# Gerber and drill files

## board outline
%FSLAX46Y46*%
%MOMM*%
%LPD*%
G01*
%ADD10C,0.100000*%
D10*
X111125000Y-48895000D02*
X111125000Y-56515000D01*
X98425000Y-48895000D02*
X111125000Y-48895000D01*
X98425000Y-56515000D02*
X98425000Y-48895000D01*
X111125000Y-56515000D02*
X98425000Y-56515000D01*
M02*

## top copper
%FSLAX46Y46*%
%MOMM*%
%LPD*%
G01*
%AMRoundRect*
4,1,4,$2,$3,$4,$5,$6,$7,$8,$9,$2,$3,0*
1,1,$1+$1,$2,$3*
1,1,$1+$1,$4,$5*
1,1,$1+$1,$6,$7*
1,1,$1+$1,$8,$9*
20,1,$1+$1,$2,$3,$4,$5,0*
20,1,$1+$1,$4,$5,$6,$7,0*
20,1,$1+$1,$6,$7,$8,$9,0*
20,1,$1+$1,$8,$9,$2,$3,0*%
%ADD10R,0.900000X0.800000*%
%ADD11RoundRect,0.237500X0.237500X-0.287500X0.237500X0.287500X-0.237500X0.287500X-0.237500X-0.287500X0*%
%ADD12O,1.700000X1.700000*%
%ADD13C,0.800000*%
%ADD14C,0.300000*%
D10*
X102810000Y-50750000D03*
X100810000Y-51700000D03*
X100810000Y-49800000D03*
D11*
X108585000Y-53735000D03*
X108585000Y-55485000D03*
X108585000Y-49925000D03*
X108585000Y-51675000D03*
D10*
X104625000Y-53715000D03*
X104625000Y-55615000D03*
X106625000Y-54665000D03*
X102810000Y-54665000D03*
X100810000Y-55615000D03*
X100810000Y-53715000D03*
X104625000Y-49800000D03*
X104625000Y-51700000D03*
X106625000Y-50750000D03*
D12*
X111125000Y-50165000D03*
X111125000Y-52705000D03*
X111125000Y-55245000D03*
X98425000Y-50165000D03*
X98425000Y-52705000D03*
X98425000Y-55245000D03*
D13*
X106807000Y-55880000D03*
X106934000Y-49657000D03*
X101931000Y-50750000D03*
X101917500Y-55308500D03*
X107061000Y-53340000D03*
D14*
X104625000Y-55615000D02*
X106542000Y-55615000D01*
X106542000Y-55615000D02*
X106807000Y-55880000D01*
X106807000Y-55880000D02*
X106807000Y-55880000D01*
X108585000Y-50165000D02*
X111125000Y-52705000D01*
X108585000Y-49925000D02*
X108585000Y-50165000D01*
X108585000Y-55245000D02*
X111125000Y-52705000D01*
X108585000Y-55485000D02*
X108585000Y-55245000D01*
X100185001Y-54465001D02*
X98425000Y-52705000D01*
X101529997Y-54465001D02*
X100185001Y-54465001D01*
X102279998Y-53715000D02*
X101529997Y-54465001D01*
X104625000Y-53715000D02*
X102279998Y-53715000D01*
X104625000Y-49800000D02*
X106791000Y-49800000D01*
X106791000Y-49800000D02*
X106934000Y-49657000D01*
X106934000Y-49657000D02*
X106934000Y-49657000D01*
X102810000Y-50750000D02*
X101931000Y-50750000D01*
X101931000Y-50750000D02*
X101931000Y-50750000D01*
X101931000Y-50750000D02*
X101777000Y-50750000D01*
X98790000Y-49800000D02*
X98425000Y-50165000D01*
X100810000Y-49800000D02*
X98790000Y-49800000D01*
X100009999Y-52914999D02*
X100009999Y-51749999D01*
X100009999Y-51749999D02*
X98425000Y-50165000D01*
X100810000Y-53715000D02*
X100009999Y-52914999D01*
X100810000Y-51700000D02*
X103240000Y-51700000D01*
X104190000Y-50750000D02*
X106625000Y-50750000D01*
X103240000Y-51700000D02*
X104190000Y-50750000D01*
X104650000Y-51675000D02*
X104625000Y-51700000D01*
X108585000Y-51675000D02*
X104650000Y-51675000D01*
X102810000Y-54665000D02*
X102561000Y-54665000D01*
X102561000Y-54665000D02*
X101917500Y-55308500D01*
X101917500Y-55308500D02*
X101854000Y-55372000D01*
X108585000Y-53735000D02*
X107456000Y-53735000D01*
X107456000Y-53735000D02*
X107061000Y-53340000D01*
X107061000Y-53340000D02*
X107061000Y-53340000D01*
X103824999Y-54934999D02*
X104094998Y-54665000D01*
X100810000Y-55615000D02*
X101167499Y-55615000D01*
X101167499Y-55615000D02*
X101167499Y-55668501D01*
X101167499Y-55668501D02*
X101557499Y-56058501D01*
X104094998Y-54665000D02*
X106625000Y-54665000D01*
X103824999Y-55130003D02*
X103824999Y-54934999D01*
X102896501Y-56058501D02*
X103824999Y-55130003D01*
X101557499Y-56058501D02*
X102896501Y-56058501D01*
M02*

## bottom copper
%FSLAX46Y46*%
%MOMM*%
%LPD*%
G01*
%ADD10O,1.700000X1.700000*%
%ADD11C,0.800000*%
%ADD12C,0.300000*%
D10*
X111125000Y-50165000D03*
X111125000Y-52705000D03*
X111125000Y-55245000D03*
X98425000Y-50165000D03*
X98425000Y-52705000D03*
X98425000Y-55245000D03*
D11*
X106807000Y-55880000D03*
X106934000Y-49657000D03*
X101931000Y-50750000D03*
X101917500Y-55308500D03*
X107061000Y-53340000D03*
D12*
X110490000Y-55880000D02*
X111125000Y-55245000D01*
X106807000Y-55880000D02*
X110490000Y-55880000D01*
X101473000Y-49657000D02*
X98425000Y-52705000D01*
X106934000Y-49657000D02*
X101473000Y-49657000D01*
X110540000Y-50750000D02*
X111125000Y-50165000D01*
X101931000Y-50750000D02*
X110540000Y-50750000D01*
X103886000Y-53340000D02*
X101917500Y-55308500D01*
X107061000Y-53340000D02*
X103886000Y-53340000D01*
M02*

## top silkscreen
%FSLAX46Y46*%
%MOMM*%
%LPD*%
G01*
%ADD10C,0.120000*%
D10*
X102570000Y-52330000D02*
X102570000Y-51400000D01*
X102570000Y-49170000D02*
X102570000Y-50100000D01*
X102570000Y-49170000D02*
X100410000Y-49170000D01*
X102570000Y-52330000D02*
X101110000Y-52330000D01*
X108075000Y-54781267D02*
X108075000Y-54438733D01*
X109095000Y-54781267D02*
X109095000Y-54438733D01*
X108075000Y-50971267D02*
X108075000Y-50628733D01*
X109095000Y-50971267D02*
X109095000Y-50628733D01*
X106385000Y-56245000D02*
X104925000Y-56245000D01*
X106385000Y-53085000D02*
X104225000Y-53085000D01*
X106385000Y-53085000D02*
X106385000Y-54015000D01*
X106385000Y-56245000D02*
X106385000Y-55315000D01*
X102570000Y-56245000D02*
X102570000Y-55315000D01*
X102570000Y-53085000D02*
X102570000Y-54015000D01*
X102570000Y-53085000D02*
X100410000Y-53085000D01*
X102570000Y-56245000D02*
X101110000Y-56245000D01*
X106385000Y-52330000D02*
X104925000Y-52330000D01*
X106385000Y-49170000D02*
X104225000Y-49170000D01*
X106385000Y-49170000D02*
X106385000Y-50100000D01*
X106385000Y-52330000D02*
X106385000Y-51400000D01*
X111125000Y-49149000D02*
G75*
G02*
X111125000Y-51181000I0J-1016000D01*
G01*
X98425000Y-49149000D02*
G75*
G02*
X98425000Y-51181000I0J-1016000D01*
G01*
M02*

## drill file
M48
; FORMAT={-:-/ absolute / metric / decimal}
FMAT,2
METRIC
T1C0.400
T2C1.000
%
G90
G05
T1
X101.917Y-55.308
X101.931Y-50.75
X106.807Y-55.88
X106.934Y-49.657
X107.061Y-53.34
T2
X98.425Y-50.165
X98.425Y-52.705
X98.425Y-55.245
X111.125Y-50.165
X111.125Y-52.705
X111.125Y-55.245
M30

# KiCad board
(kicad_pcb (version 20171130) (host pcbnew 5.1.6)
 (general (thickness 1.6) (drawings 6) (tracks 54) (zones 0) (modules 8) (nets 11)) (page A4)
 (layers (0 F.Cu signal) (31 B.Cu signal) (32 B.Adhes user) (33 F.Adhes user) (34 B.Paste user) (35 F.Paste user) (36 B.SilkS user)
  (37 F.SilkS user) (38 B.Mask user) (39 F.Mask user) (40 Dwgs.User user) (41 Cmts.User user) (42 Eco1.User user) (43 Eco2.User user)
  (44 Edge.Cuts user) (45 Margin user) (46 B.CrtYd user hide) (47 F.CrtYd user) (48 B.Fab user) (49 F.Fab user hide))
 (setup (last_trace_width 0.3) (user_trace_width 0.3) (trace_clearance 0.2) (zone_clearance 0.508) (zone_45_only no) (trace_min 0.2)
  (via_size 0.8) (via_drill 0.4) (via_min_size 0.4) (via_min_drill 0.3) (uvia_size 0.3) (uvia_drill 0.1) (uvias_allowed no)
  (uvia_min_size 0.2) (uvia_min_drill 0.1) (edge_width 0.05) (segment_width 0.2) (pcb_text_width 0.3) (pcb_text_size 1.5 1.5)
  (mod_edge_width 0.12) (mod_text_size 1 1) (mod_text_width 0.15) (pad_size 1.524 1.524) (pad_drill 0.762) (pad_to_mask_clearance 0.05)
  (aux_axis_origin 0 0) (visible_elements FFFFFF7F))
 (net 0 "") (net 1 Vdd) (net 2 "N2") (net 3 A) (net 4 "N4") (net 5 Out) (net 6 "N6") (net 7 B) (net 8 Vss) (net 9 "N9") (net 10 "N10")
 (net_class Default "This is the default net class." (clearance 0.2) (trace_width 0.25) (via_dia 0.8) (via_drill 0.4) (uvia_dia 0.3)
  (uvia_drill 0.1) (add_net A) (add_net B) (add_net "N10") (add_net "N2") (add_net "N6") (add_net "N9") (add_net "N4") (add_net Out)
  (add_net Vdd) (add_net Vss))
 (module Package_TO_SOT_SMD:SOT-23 (layer F.Cu) (at 101.81 50.75)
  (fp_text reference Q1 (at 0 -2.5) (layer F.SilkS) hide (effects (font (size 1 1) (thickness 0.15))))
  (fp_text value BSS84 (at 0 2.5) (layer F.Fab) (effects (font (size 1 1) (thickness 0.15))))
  (fp_line (start 0.76 1.58) (end 0.76 0.65) (layer F.SilkS) (width 0.12))
  (fp_line (start 0.76 -1.58) (end 0.76 -0.65) (layer F.SilkS) (width 0.12))
  (fp_line (start 0.76 -1.58) (end -1.4 -1.58) (layer F.SilkS) (width 0.12))
  (fp_line (start 0.76 1.58) (end -0.7 1.58) (layer F.SilkS) (width 0.12))
  (pad 3 smd rect (at 1 0) (size 0.9 0.8) (layers F.Cu F.Paste F.Mask) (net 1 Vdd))
  (pad 2 smd rect (at -1 0.95) (size 0.9 0.8) (layers F.Cu F.Paste F.Mask) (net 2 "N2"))
  (pad 1 smd rect (at -1 -0.95) (size 0.9 0.8) (layers F.Cu F.Paste F.Mask) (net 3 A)))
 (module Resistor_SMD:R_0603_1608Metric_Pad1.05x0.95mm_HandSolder (layer F.Cu) (at 108.585 54.61 90)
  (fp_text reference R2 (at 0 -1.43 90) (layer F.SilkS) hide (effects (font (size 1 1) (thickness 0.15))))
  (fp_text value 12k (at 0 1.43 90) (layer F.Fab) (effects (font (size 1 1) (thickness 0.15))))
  (fp_line (start -0.171267 -0.51) (end 0.171267 -0.51) (layer F.SilkS) (width 0.12))
  (fp_line (start -0.171267 0.51) (end 0.171267 0.51) (layer F.SilkS) (width 0.12))
  (pad 2 smd roundrect (at 0.875 0 90) (size 1.05 0.95) (layers F.Cu F.Paste F.Mask) (roundrect_rratio 0.25) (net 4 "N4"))
  (pad 1 smd roundrect (at -0.875 0 90) (size 1.05 0.95) (layers F.Cu F.Paste F.Mask) (roundrect_rratio 0.25) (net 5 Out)))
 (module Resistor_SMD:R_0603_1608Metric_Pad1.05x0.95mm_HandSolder (layer F.Cu) (at 108.585 50.8 90)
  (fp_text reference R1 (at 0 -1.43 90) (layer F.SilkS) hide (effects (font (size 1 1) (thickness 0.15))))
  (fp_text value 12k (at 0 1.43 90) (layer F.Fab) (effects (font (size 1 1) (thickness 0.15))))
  (fp_line (start -0.171267 -0.51) (end 0.171267 -0.51) (layer F.SilkS) (width 0.12))
  (fp_line (start -0.171267 0.51) (end 0.171267 0.51) (layer F.SilkS) (width 0.12))
  (pad 2 smd roundrect (at 0.875 0 90) (size 1.05 0.95) (layers F.Cu F.Paste F.Mask) (roundrect_rratio 0.25) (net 5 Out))
  (pad 1 smd roundrect (at -0.875 0 90) (size 1.05 0.95) (layers F.Cu F.Paste F.Mask) (roundrect_rratio 0.25) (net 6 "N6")))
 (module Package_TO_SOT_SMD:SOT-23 (layer F.Cu) (at 105.625 54.665)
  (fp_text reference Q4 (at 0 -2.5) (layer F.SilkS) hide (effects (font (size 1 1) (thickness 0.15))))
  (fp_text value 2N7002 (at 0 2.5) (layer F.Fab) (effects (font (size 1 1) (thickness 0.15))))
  (fp_line (start 0.76 1.58) (end -0.7 1.58) (layer F.SilkS) (width 0.12))
  (fp_line (start 0.76 -1.58) (end -1.4 -1.58) (layer F.SilkS) (width 0.12))
  (fp_line (start 0.76 -1.58) (end 0.76 -0.65) (layer F.SilkS) (width 0.12))
  (fp_line (start 0.76 1.58) (end 0.76 0.65) (layer F.SilkS) (width 0.12))
  (pad 1 smd rect (at -1 -0.95) (size 0.9 0.8) (layers F.Cu F.Paste F.Mask) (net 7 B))
  (pad 2 smd rect (at -1 0.95) (size 0.9 0.8) (layers F.Cu F.Paste F.Mask) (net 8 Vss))
  (pad 3 smd rect (at 1 0) (size 0.9 0.8) (layers F.Cu F.Paste F.Mask) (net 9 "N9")))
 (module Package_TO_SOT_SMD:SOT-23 (layer F.Cu) (at 101.81 54.665)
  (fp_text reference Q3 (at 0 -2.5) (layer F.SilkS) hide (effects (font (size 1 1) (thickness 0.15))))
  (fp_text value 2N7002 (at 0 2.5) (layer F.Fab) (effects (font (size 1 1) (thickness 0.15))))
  (fp_line (start 0.76 1.58) (end 0.76 0.65) (layer F.SilkS) (width 0.12))
  (fp_line (start 0.76 -1.58) (end 0.76 -0.65) (layer F.SilkS) (width 0.12))
  (fp_line (start 0.76 -1.58) (end -1.4 -1.58) (layer F.SilkS) (width 0.12))
  (fp_line (start 0.76 1.58) (end -0.7 1.58) (layer F.SilkS) (width 0.12))
  (pad 3 smd rect (at 1 0) (size 0.9 0.8) (layers F.Cu F.Paste F.Mask) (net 4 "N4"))
  (pad 2 smd rect (at -1 0.95) (size 0.9 0.8) (layers F.Cu F.Paste F.Mask) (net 9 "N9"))
  (pad 1 smd rect (at -1 -0.95) (size 0.9 0.8) (layers F.Cu F.Paste F.Mask) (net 3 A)))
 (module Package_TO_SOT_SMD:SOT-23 (layer F.Cu) (at 105.625 50.75)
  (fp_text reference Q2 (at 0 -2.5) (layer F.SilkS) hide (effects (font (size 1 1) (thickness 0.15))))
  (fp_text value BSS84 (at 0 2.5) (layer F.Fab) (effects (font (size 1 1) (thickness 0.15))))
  (fp_line (start 0.76 1.58) (end -0.7 1.58) (layer F.SilkS) (width 0.12))
  (fp_line (start 0.76 -1.58) (end -1.4 -1.58) (layer F.SilkS) (width 0.12))
  (fp_line (start 0.76 -1.58) (end 0.76 -0.65) (layer F.SilkS) (width 0.12))
  (fp_line (start 0.76 1.58) (end 0.76 0.65) (layer F.SilkS) (width 0.12))
  (pad 1 smd rect (at -1 -0.95) (size 0.9 0.8) (layers F.Cu F.Paste F.Mask) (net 7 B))
  (pad 2 smd rect (at -1 0.95) (size 0.9 0.8) (layers F.Cu F.Paste F.Mask) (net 6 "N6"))
  (pad 3 smd rect (at 1 0) (size 0.9 0.8) (layers F.Cu F.Paste F.Mask) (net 2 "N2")))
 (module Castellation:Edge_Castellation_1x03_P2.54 (layer F.Cu) (at 111.125 50.165)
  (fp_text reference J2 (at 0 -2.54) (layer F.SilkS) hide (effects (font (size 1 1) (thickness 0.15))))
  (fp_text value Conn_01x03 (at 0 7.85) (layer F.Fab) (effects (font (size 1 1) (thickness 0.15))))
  (fp_arc (start 0 0) (end 0 1.016) (angle -180) (layer F.SilkS) (width 0.12))
  (pad 1 thru_hole oval (at 0 0) (size 1.7 1.7) (drill 1) (layers *.Cu *.Mask) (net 1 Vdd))
  (pad 2 thru_hole oval (at 0 2.54) (size 1.7 1.7) (drill 1) (layers *.Cu *.Mask) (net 5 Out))
  (pad 3 thru_hole oval (at 0 5.08) (size 1.7 1.7) (drill 1) (layers *.Cu *.Mask) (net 8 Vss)))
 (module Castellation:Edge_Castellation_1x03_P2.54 (layer F.Cu) (at 98.425 50.165)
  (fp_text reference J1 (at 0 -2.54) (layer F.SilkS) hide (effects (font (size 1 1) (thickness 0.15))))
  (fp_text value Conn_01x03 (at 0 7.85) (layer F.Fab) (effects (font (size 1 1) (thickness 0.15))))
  (fp_arc (start 0 0) (end 0 1.016) (angle -180) (layer F.SilkS) (width 0.12))
  (pad 1 thru_hole oval (at 0 0) (size 1.7 1.7) (drill 1) (layers *.Cu *.Mask) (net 3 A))
  (pad 2 thru_hole oval (at 0 2.54) (size 1.7 1.7) (drill 1) (layers *.Cu *.Mask) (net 7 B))
  (pad 3 thru_hole oval (at 0 5.08) (size 1.7 1.7) (drill 1) (layers *.Cu *.Mask) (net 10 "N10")))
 (gr_line (start 111.125 48.895) (end 111.125 56.515) (layer Edge.Cuts) (width 0.1))
 (gr_line (start 98.425 48.895) (end 111.125 48.895) (layer Edge.Cuts) (width 0.1))
 (gr_line (start 98.425 56.515) (end 98.425 48.895) (layer Edge.Cuts) (width 0.1))
 (gr_line (start 111.125 56.515) (end 98.425 56.515) (layer Edge.Cuts) (width 0.1))
 (segment (start 104.625 55.615) (end 106.542 55.615) (width 0.3) (layer F.Cu) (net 8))
 (segment (start 106.542 55.615) (end 106.807 55.88) (width 0.3) (layer F.Cu) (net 8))
 (segment (start 106.807 55.88) (end 106.807 55.88) (width 0.3) (layer F.Cu) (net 8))
 (via (at 106.807 55.88) (size 0.8) (drill 0.4) (layers F.Cu B.Cu) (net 8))
 (segment (start 110.49 55.88) (end 111.125 55.245) (width 0.3) (layer B.Cu) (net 8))
 (segment (start 106.807 55.88) (end 110.49 55.88) (width 0.3) (layer B.Cu) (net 8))
 (segment (start 108.585 50.165) (end 111.125 52.705) (width 0.3) (layer F.Cu) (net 5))
 (segment (start 108.585 49.925) (end 108.585 50.165) (width 0.3) (layer F.Cu) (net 5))
 (segment (start 108.585 55.245) (end 111.125 52.705) (width 0.3) (layer F.Cu) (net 5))
 (segment (start 108.585 55.485) (end 108.585 55.245) (width 0.3) (layer F.Cu) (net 5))
 (segment (start 100.185001 54.465001) (end 98.425 52.705) (width 0.3) (layer F.Cu) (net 7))
 (segment (start 101.529997 54.465001) (end 100.185001 54.465001) (width 0.3) (layer F.Cu) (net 7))
 (segment (start 102.279998 53.715) (end 101.529997 54.465001) (width 0.3) (layer F.Cu) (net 7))
 (segment (start 104.625 53.715) (end 102.279998 53.715) (width 0.3) (layer F.Cu) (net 7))
 (segment (start 104.625 49.8) (end 106.791 49.8) (width 0.3) (layer F.Cu) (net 7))
 (segment (start 106.791 49.8) (end 106.934 49.657) (width 0.3) (layer F.Cu) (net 7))
 (segment (start 106.934 49.657) (end 106.934 49.657) (width 0.3) (layer F.Cu) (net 7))
 (via (at 106.934 49.657) (size 0.8) (drill 0.4) (layers F.Cu B.Cu) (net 7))
 (segment (start 101.473 49.657) (end 98.425 52.705) (width 0.3) (layer B.Cu) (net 7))
 (segment (start 106.934 49.657) (end 101.473 49.657) (width 0.3) (layer B.Cu) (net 7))
 (segment (start 102.81 50.75) (end 101.931 50.75) (width 0.3) (layer F.Cu) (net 1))
 (segment (start 101.931 50.75) (end 101.931 50.75) (width 0.3) (layer F.Cu) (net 1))
 (segment (start 101.931 50.75) (end 101.777 50.75) (width 0.3) (layer F.Cu) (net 1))
 (via (at 101.931 50.75) (size 0.8) (drill 0.4) (layers F.Cu B.Cu) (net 1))
 (segment (start 110.54 50.75) (end 111.125 50.165) (width 0.3) (layer B.Cu) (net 1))
 (segment (start 101.931 50.75) (end 110.54 50.75) (width 0.3) (layer B.Cu) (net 1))
 (segment (start 98.79 49.8) (end 98.425 50.165) (width 0.3) (layer F.Cu) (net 3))
 (segment (start 100.81 49.8) (end 98.79 49.8) (width 0.3) (layer F.Cu) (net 3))
 (segment (start 100.009999 52.914999) (end 100.009999 51.749999) (width 0.3) (layer F.Cu) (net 3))
 (segment (start 100.009999 51.749999) (end 98.425 50.165) (width 0.3) (layer F.Cu) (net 3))
 (segment (start 100.81 53.715) (end 100.009999 52.914999) (width 0.3) (layer F.Cu) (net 3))
 (segment (start 100.81 51.7) (end 103.24 51.7) (width 0.3) (layer F.Cu) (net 2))
 (segment (start 104.19 50.75) (end 106.625 50.75) (width 0.3) (layer F.Cu) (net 2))
 (segment (start 103.24 51.7) (end 104.19 50.75) (width 0.3) (layer F.Cu) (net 2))
 (segment (start 104.65 51.675) (end 104.625 51.7) (width 0.3) (layer F.Cu) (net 6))
 (segment (start 108.585 51.675) (end 104.65 51.675) (width 0.3) (layer F.Cu) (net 6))
 (segment (start 102.81 54.665) (end 102.561 54.665) (width 0.3) (layer F.Cu) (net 4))
 (segment (start 102.561 54.665) (end 101.9175 55.3085) (width 0.3) (layer F.Cu) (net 4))
 (segment (start 101.9175 55.3085) (end 101.854 55.372) (width 0.3) (layer F.Cu) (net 4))
 (via (at 101.9175 55.3085) (size 0.8) (drill 0.4) (layers F.Cu B.Cu) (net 4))
 (segment (start 108.585 53.735) (end 107.456 53.735) (width 0.3) (layer F.Cu) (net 4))
 (segment (start 107.456 53.735) (end 107.061 53.34) (width 0.3) (layer F.Cu) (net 4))
 (segment (start 107.061 53.34) (end 107.061 53.34) (width 0.3) (layer F.Cu) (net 4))
 (via (at 107.061 53.34) (size 0.8) (drill 0.4) (layers F.Cu B.Cu) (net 4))
 (segment (start 103.886 53.34) (end 101.9175 55.3085) (width 0.3) (layer B.Cu) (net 4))
 (segment (start 107.061 53.34) (end 103.886 53.34) (width 0.3) (layer B.Cu) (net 4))
 (segment (start 103.824999 54.934999) (end 104.094998 54.665) (width 0.3) (layer F.Cu) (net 9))
 (segment (start 100.81 55.615) (end 101.167499 55.615) (width 0.3) (layer F.Cu) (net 9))
 (segment (start 101.167499 55.615) (end 101.167499 55.668501) (width 0.3) (layer F.Cu) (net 9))
 (segment (start 101.167499 55.668501) (end 101.557499 56.058501) (width 0.3) (layer F.Cu) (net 9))
 (segment (start 104.094998 54.665) (end 106.625 54.665) (width 0.3) (layer F.Cu) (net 9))
 (segment (start 103.824999 55.130003) (end 103.824999 54.934999) (width 0.3) (layer F.Cu) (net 9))
 (segment (start 102.896501 56.058501) (end 103.824999 55.130003) (width 0.3) (layer F.Cu) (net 9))
 (segment (start 101.557499 56.058501) (end 102.896501 56.058501) (width 0.3) (layer F.Cu) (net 9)))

